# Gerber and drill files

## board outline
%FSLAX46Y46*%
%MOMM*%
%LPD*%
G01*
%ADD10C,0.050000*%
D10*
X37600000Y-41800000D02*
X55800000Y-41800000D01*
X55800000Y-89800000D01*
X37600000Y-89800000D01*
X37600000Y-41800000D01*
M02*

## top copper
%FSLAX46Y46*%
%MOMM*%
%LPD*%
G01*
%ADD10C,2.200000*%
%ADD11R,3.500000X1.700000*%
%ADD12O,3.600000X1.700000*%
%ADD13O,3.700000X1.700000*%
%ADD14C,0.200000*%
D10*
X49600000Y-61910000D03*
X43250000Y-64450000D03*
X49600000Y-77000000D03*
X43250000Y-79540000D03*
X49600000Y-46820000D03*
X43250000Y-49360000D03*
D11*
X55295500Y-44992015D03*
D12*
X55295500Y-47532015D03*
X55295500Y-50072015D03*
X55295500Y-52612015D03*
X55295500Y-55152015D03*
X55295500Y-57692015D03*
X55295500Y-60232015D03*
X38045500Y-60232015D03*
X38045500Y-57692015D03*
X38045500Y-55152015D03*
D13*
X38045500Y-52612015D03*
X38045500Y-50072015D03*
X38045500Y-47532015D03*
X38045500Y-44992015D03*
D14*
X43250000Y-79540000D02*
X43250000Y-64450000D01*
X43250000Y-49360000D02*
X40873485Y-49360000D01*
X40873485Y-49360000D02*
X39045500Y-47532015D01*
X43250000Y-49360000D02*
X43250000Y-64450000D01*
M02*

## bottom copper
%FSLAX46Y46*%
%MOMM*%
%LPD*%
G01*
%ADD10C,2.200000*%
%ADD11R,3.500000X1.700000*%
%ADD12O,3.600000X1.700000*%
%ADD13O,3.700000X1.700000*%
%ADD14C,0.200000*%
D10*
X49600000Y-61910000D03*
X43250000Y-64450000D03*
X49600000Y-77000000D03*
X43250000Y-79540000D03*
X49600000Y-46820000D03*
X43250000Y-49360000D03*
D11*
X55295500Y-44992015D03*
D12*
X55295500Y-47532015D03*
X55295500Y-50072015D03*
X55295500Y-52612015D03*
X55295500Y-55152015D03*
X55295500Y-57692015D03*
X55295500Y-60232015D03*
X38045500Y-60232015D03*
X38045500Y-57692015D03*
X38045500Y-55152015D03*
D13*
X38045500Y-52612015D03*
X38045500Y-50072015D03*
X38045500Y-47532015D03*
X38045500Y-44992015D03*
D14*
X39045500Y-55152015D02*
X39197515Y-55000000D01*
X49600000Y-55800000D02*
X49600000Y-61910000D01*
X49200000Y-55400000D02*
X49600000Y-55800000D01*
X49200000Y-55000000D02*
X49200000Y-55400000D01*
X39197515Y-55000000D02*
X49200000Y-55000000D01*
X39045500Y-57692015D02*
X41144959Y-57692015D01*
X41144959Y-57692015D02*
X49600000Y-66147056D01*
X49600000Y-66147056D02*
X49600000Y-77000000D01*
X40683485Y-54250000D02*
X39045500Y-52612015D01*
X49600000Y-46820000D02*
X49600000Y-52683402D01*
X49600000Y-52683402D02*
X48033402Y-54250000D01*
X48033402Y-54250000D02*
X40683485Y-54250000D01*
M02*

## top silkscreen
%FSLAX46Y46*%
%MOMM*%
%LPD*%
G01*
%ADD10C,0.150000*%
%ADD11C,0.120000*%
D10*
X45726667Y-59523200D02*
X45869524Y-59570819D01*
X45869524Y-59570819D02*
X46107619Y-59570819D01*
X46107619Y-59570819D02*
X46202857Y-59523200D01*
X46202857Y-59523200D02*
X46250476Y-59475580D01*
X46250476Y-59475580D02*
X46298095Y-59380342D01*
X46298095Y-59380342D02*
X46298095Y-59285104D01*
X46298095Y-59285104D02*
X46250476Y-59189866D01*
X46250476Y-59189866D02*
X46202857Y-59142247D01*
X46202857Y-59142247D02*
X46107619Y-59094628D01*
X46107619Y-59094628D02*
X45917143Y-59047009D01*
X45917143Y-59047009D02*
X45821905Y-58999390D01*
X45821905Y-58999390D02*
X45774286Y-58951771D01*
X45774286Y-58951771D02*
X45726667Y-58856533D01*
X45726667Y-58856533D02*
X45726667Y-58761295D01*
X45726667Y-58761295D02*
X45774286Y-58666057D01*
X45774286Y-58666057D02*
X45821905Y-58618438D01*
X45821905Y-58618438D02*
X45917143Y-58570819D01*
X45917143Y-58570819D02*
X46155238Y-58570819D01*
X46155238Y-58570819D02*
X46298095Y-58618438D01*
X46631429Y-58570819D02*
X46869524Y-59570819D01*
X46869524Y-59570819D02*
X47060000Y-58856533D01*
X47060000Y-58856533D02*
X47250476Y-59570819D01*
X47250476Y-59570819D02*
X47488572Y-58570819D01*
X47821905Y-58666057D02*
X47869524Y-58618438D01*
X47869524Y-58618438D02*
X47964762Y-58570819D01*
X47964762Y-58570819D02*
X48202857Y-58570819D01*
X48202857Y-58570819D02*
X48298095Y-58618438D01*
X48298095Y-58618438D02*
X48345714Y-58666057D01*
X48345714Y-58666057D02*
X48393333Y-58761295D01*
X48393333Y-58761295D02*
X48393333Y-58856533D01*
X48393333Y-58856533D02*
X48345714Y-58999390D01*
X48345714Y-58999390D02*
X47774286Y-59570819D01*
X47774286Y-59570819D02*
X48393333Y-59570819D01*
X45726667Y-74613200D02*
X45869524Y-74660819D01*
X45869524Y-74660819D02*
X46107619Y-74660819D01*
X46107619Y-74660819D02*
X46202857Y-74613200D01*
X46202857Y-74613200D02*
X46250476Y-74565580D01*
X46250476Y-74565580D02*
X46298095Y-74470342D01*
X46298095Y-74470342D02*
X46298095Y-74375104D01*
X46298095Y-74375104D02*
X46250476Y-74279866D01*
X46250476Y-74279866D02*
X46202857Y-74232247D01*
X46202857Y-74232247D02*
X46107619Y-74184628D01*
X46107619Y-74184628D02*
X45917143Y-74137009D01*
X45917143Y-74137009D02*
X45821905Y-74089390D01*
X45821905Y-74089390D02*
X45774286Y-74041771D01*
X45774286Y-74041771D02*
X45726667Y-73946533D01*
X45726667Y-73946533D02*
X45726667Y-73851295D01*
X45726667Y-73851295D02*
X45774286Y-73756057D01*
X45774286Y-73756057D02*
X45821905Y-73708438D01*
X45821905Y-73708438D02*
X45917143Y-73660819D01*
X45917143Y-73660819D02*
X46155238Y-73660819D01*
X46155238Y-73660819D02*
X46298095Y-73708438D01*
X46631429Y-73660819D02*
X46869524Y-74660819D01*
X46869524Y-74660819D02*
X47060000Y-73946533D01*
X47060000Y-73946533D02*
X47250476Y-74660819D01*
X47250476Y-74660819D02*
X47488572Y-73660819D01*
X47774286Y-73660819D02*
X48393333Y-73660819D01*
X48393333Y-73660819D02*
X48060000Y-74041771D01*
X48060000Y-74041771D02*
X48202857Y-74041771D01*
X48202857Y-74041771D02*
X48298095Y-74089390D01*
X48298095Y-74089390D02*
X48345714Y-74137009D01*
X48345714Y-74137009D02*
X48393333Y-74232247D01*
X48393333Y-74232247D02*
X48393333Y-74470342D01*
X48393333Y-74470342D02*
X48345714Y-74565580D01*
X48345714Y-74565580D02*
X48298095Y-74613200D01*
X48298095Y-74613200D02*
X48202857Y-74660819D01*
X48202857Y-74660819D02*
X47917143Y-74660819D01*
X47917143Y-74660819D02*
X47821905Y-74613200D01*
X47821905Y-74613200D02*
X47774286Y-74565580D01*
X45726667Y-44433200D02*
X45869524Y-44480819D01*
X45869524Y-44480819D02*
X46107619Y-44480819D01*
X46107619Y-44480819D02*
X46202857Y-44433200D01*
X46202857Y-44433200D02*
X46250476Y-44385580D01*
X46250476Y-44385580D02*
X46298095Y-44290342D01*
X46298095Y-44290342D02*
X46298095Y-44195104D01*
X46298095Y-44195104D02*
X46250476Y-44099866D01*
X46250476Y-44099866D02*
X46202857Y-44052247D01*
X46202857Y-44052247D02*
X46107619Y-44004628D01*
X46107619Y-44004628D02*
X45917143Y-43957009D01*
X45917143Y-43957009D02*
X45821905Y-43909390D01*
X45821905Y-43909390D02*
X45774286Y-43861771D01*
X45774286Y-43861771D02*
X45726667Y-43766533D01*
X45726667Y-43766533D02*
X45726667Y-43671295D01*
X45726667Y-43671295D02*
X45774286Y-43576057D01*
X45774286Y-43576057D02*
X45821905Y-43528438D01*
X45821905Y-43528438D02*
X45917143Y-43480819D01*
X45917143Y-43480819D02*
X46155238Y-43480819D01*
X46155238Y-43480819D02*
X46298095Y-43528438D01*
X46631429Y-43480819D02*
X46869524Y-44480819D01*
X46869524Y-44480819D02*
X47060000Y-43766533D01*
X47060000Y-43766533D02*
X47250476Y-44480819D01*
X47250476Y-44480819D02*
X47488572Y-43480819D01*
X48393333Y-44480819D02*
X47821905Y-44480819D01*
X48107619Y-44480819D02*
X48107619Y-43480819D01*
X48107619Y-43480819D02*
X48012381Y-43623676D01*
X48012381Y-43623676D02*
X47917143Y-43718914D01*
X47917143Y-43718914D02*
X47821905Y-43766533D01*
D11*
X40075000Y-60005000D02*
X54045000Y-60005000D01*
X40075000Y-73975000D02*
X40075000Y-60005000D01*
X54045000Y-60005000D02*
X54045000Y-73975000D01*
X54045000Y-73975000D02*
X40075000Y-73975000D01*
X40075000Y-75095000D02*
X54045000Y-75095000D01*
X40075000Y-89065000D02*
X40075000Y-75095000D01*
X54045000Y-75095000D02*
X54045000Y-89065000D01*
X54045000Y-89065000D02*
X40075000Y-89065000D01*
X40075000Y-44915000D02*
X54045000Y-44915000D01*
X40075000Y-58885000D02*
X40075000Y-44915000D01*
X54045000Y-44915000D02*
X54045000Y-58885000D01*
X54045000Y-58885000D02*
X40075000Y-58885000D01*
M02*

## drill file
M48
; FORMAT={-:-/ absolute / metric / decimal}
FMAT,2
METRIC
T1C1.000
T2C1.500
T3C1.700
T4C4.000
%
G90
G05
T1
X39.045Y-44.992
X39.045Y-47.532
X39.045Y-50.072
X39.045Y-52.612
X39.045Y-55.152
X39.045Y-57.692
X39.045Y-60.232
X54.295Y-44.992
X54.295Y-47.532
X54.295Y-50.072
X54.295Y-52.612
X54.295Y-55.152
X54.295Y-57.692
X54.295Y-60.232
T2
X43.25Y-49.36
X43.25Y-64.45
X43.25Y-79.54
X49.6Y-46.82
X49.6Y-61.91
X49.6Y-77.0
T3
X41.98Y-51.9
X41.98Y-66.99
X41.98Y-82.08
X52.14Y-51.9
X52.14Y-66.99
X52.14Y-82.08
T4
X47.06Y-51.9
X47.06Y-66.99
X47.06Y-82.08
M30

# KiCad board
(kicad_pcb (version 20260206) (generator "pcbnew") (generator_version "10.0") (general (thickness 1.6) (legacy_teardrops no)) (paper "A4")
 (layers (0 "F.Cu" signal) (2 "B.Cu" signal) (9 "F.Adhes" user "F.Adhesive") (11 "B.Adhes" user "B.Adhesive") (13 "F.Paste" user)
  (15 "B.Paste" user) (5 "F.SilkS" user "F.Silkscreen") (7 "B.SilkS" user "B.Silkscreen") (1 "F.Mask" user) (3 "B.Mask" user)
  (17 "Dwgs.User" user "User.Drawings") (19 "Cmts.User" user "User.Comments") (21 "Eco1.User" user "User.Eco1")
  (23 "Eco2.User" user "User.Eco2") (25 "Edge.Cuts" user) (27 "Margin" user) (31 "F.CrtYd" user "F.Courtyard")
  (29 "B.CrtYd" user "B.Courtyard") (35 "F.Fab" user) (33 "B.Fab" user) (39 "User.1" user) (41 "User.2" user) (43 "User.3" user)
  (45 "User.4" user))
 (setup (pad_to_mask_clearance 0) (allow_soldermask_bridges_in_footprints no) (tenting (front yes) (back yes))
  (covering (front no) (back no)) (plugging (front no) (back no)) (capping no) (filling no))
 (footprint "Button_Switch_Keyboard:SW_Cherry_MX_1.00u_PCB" (layer "F.Cu") (at 49.6 61.91)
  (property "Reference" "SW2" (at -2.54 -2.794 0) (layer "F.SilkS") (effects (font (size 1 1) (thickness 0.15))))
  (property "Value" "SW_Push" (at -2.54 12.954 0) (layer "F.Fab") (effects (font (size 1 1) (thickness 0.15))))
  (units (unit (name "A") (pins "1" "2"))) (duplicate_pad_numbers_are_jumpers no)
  (fp_line (start -9.525 -1.905) (end 4.445 -1.905) (stroke (width 0.12) (type solid)) (layer "F.SilkS"))
  (fp_line (start -9.525 12.065) (end -9.525 -1.905) (stroke (width 0.12) (type solid)) (layer "F.SilkS"))
  (fp_line (start 4.445 -1.905) (end 4.445 12.065) (stroke (width 0.12) (type solid)) (layer "F.SilkS"))
  (fp_line (start 4.445 12.065) (end -9.525 12.065) (stroke (width 0.12) (type solid)) (layer "F.SilkS"))
  (pad "" np_thru_hole circle (at -7.62 5.08) (size 1.7 1.7) (drill 1.7) (layers "*.Cu" "*.Mask"))
  (pad "" np_thru_hole circle (at -2.54 5.08) (size 4 4) (drill 4) (layers "*.Cu" "*.Mask"))
  (pad "" np_thru_hole circle (at 2.54 5.08) (size 1.7 1.7) (drill 1.7) (layers "*.Cu" "*.Mask"))
  (pad "1" thru_hole circle (at 0 0) (size 2.2 2.2) (drill 1.5) (layers "*.Cu" "*.Mask") (remove_unused_layers no)
   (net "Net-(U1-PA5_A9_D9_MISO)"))
  (pad "2" thru_hole circle (at -6.35 2.54) (size 2.2 2.2) (drill 1.5) (layers "*.Cu" "*.Mask") (remove_unused_layers no) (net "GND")))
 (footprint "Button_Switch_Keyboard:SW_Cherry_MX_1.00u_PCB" (layer "F.Cu") (at 49.6 77)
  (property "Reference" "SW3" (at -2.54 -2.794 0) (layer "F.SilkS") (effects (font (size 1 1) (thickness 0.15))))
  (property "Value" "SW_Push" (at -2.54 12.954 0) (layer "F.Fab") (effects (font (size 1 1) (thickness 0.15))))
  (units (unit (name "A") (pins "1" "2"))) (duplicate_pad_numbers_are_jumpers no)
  (fp_line (start -9.525 -1.905) (end 4.445 -1.905) (stroke (width 0.12) (type solid)) (layer "F.SilkS"))
  (fp_line (start -9.525 12.065) (end -9.525 -1.905) (stroke (width 0.12) (type solid)) (layer "F.SilkS"))
  (fp_line (start 4.445 -1.905) (end 4.445 12.065) (stroke (width 0.12) (type solid)) (layer "F.SilkS"))
  (fp_line (start 4.445 12.065) (end -9.525 12.065) (stroke (width 0.12) (type solid)) (layer "F.SilkS"))
  (pad "" np_thru_hole circle (at -7.62 5.08) (size 1.7 1.7) (drill 1.7) (layers "*.Cu" "*.Mask"))
  (pad "" np_thru_hole circle (at -2.54 5.08) (size 4 4) (drill 4) (layers "*.Cu" "*.Mask"))
  (pad "" np_thru_hole circle (at 2.54 5.08) (size 1.7 1.7) (drill 1.7) (layers "*.Cu" "*.Mask"))
  (pad "1" thru_hole circle (at 0 0) (size 2.2 2.2) (drill 1.5) (layers "*.Cu" "*.Mask") (remove_unused_layers no)
   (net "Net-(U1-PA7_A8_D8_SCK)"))
  (pad "2" thru_hole circle (at -6.35 2.54) (size 2.2 2.2) (drill 1.5) (layers "*.Cu" "*.Mask") (remove_unused_layers no) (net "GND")))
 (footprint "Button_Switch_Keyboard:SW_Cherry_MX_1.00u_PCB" (layer "F.Cu") (at 49.6 46.82)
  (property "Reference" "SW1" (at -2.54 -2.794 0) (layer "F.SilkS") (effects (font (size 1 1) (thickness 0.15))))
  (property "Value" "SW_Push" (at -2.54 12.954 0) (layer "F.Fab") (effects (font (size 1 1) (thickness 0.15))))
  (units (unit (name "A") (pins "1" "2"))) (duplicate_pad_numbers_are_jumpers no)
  (fp_line (start -9.525 -1.905) (end 4.445 -1.905) (stroke (width 0.12) (type solid)) (layer "F.SilkS"))
  (fp_line (start -9.525 12.065) (end -9.525 -1.905) (stroke (width 0.12) (type solid)) (layer "F.SilkS"))
  (fp_line (start 4.445 -1.905) (end 4.445 12.065) (stroke (width 0.12) (type solid)) (layer "F.SilkS"))
  (fp_line (start 4.445 12.065) (end -9.525 12.065) (stroke (width 0.12) (type solid)) (layer "F.SilkS"))
  (pad "" np_thru_hole circle (at -7.62 5.08) (size 1.7 1.7) (drill 1.7) (layers "*.Cu" "*.Mask"))
  (pad "" np_thru_hole circle (at -2.54 5.08) (size 4 4) (drill 4) (layers "*.Cu" "*.Mask"))
  (pad "" np_thru_hole circle (at 2.54 5.08) (size 1.7 1.7) (drill 1.7) (layers "*.Cu" "*.Mask"))
  (pad "1" thru_hole circle (at 0 0) (size 2.2 2.2) (drill 1.5) (layers "*.Cu" "*.Mask") (remove_unused_layers no)
   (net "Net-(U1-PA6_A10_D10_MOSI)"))
  (pad "2" thru_hole circle (at -6.35 2.54) (size 2.2 2.2) (drill 1.5) (layers "*.Cu" "*.Mask") (remove_unused_layers no) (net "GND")))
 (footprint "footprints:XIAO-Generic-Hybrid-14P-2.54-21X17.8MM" (layer "B.Cu") (at 46.6705 52.612015 180)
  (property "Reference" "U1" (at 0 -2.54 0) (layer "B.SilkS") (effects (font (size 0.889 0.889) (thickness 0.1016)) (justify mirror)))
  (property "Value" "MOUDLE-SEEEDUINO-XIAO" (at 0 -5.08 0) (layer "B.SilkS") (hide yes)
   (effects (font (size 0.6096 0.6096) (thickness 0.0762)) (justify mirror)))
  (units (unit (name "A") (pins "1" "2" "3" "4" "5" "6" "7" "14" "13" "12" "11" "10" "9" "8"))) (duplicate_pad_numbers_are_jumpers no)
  (pad "1" thru_hole rect (at -7.625 7.62 180) (size 3.5 1.7) (drill 1 (offset -1 0)) (layers "*.Cu" "*.Mask") (remove_unused_layers no)
   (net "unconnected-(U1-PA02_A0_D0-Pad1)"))
  (pad "2" thru_hole oval (at -7.625 5.08 180) (size 3.6 1.7) (drill 1 (offset -1 0)) (layers "*.Cu" "*.Mask") (remove_unused_layers no)
   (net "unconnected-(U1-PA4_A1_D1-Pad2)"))
  (pad "3" thru_hole oval (at -7.625 2.54 180) (size 3.6 1.7) (drill 1 (offset -1 0)) (layers "*.Cu" "*.Mask") (remove_unused_layers no)
   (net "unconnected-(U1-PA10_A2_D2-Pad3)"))
  (pad "4" thru_hole oval (at -7.625 0 180) (size 3.6 1.7) (drill 1 (offset -1 0)) (layers "*.Cu" "*.Mask") (remove_unused_layers no)
   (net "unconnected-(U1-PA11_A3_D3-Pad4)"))
  (pad "5" thru_hole oval (at -7.625 -2.54 180) (size 3.6 1.7) (drill 1 (offset -1 0)) (layers "*.Cu" "*.Mask") (remove_unused_layers no)
   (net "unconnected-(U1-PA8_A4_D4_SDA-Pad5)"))
  (pad "6" thru_hole oval (at -7.625 -5.08) (size 3.6 1.7) (drill 1 (offset 1 0)) (layers "*.Cu" "*.Mask") (remove_unused_layers no)
   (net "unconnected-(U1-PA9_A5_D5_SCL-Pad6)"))
  (pad "7" thru_hole oval (at -7.625 -7.62 180) (size 3.6 1.7) (drill 1 (offset -1 0)) (layers "*.Cu" "*.Mask") (remove_unused_layers no)
   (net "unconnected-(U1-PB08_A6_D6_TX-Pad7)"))
  (pad "8" thru_hole oval (at 7.625 -7.62 180) (size 3.6 1.7) (drill 1 (offset 1 0)) (layers "*.Cu" "*.Mask") (remove_unused_layers no)
   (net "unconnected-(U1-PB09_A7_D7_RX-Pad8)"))
  (pad "9" thru_hole oval (at 7.625 -5.08 180) (size 3.6 1.7) (drill 1 (offset 1 0)) (layers "*.Cu" "*.Mask") (remove_unused_layers no)
   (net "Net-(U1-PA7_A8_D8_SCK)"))
  (pad "10" thru_hole oval (at 7.625 -2.54 180) (size 3.6 1.7) (drill 1 (offset 1 0)) (layers "*.Cu" "*.Mask") (remove_unused_layers no)
   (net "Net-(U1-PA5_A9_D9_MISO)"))
  (pad "11" thru_hole oval (at 7.625 0 180) (size 3.7 1.7) (drill 1 (offset 1 0)) (layers "*.Cu" "*.Mask") (remove_unused_layers no)
   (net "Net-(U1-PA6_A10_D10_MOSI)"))
  (pad "12" thru_hole oval (at 7.625 2.54 180) (size 3.7 1.7) (drill 1 (offset 1 0)) (layers "*.Cu" "*.Mask") (remove_unused_layers no)
   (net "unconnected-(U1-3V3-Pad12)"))
  (pad "13" thru_hole oval (at 7.625 5.08 180) (size 3.7 1.7) (drill 1 (offset 1 0)) (layers "*.Cu" "*.Mask") (remove_unused_layers no)
   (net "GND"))
  (pad "14" thru_hole oval (at 7.625 7.62 180) (size 3.7 1.7) (drill 1 (offset 1 0)) (layers "*.Cu" "*.Mask") (remove_unused_layers no)
   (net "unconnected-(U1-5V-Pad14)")))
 (gr_rect (start 37.6 41.8) (end 55.8 89.8) (stroke (width 0.05) (type default)) (fill no) (layer "Edge.Cuts"))
 (segment (start 39.0455 55.152015) (end 39.197515 55) (width 0.2) (layer "B.Cu") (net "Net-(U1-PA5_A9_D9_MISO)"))
 (segment (start 49.6 55.8) (end 49.6 61.91) (width 0.2) (layer "B.Cu") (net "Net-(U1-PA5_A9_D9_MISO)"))
 (segment (start 49.2 55.4) (end 49.6 55.8) (width 0.2) (layer "B.Cu") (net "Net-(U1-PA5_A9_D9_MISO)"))
 (segment (start 49.2 55) (end 49.2 55.4) (width 0.2) (layer "B.Cu") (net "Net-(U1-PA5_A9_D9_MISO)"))
 (segment (start 39.197515 55) (end 49.2 55) (width 0.2) (layer "B.Cu") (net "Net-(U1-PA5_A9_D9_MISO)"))
 (segment (start 43.25 79.54) (end 43.25 64.45) (width 0.2) (layer "F.Cu") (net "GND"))
 (segment (start 43.25 49.36) (end 40.873485 49.36) (width 0.2) (layer "F.Cu") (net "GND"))
 (segment (start 40.873485 49.36) (end 39.0455 47.532015) (width 0.2) (layer "F.Cu") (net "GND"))
 (segment (start 43.25 49.36) (end 43.25 64.45) (width 0.2) (layer "F.Cu") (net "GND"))
 (segment (start 39.0455 57.692015) (end 41.144959 57.692015) (width 0.2) (layer "B.Cu") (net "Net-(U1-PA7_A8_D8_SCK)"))
 (segment (start 41.144959 57.692015) (end 49.6 66.147056) (width 0.2) (layer "B.Cu") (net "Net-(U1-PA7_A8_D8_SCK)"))
 (segment (start 49.6 66.147056) (end 49.6 77) (width 0.2) (layer "B.Cu") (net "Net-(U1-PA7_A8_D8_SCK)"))
 (segment (start 40.683485 54.25) (end 39.0455 52.612015) (width 0.2) (layer "B.Cu") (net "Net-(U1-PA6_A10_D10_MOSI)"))
 (segment (start 49.6 46.82) (end 49.6 52.683402) (width 0.2) (layer "B.Cu") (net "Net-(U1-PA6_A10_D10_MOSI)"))
 (segment (start 49.6 52.683402) (end 48.033402 54.25) (width 0.2) (layer "B.Cu") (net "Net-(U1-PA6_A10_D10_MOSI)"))
 (segment (start 48.033402 54.25) (end 40.683485 54.25) (width 0.2) (layer "B.Cu") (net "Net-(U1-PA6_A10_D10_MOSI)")))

